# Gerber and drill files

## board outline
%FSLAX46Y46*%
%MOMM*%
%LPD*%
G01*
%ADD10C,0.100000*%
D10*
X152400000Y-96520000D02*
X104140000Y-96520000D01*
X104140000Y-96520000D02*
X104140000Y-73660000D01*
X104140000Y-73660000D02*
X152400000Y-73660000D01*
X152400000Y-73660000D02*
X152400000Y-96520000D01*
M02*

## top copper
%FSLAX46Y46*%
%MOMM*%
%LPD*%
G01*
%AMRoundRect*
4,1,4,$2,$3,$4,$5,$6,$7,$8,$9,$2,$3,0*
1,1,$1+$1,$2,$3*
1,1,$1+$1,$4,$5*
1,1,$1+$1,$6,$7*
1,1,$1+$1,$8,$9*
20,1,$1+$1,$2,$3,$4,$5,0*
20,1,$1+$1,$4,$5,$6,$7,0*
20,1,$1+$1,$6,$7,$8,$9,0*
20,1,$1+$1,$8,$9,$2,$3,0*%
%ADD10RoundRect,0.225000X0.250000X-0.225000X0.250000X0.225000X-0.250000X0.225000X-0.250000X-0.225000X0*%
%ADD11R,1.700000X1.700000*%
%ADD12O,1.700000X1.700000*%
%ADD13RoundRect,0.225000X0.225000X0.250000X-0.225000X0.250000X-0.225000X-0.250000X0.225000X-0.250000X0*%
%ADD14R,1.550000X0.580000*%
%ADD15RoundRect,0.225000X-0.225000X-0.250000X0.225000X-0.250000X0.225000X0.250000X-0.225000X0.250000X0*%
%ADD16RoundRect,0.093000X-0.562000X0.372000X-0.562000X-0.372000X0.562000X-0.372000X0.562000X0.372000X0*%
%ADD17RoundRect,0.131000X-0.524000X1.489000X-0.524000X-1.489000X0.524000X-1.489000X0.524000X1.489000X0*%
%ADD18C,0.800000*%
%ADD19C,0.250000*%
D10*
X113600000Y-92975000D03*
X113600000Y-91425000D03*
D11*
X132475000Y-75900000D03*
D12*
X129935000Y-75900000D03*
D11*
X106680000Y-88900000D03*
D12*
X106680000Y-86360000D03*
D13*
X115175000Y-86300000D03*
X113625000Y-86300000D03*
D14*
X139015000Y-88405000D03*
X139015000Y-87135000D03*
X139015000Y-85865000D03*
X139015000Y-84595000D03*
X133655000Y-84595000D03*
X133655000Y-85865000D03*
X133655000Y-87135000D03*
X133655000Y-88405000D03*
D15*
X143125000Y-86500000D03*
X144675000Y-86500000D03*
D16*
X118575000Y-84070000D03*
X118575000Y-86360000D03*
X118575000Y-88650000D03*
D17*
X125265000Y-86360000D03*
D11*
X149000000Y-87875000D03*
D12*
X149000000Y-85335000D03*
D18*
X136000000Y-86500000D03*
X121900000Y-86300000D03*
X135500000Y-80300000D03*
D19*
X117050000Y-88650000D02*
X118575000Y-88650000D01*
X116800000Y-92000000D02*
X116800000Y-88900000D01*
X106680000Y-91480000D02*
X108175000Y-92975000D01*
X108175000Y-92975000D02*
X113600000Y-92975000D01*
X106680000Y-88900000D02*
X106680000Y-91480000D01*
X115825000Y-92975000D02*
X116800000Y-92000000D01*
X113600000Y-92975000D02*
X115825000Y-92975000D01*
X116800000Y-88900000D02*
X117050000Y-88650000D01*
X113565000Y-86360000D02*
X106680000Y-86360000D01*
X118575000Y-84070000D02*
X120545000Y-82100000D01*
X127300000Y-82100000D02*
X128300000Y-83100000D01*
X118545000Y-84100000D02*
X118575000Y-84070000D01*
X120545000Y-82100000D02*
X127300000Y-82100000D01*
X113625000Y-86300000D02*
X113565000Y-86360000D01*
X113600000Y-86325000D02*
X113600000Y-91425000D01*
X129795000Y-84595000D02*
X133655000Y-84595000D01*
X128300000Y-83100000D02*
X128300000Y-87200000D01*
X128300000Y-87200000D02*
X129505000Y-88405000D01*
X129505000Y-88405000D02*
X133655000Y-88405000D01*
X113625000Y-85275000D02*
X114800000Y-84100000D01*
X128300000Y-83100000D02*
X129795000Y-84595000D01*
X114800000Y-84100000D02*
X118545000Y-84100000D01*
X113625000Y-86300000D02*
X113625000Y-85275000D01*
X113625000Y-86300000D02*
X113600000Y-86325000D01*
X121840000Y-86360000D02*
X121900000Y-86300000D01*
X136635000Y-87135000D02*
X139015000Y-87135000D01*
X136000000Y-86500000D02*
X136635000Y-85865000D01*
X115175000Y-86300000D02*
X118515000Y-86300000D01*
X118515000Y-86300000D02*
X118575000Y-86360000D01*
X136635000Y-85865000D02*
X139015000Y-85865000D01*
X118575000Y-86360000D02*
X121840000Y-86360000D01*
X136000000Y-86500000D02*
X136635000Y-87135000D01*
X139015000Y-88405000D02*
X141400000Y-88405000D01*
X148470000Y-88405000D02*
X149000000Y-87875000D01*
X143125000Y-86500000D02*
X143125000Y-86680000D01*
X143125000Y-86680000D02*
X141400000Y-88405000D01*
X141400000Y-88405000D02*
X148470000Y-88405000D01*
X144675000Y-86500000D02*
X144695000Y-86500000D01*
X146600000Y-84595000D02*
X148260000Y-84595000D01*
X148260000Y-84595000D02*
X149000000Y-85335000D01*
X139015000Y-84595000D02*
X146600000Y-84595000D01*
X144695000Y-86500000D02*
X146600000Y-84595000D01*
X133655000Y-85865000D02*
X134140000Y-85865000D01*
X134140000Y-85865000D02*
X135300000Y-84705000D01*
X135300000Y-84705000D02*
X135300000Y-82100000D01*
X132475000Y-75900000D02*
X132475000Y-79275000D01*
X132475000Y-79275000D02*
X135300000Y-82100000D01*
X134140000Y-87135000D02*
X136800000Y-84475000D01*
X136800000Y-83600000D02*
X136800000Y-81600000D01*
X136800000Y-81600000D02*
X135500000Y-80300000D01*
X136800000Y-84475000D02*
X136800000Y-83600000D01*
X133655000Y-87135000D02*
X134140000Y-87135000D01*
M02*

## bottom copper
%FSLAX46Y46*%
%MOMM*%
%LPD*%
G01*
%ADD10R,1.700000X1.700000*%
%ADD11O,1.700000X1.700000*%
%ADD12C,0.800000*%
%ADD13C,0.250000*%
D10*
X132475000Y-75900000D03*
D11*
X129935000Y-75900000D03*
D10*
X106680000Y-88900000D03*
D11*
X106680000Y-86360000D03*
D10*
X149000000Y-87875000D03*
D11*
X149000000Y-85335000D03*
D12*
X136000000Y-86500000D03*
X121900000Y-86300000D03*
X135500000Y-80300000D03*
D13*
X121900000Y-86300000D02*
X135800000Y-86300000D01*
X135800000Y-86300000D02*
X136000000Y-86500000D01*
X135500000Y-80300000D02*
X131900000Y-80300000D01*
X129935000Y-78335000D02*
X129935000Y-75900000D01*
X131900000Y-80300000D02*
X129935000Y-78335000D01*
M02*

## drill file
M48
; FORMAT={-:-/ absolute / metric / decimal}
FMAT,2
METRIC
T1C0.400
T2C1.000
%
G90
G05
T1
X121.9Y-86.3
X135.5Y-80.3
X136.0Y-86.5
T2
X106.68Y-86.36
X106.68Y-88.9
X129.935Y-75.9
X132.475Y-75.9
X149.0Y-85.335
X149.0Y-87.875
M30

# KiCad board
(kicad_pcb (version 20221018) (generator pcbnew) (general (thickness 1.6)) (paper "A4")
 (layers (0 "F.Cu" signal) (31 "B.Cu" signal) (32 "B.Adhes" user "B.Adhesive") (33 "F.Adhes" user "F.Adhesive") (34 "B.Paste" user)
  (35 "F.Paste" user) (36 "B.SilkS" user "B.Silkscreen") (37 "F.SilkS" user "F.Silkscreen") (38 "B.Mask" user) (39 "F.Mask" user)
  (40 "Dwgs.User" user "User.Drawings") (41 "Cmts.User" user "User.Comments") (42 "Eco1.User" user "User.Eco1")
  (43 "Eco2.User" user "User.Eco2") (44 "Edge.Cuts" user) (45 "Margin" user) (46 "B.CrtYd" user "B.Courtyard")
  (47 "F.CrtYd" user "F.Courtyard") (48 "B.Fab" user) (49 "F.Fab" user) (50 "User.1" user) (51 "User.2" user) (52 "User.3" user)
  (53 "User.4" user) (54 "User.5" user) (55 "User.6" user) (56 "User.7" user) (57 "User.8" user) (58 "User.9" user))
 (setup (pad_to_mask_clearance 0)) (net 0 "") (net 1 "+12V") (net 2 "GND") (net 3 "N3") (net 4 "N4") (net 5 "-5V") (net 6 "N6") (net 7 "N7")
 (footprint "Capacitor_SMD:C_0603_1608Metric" (layer "F.Cu") (at 113.6 92.2 90)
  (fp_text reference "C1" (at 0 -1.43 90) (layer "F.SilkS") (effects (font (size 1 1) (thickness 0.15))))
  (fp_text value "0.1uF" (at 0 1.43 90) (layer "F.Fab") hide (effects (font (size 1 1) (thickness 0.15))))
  (pad "1" smd roundrect (at -0.775 0 90) (size 0.9 0.95) (layers "F.Cu" "F.Paste" "F.Mask") (roundrect_rratio 0.25) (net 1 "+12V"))
  (pad "2" smd roundrect (at 0.775 0 90) (size 0.9 0.95) (layers "F.Cu" "F.Paste" "F.Mask") (roundrect_rratio 0.25) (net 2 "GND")))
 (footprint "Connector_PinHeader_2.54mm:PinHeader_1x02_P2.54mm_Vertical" (layer "F.Cu") (at 132.475 75.9 -90)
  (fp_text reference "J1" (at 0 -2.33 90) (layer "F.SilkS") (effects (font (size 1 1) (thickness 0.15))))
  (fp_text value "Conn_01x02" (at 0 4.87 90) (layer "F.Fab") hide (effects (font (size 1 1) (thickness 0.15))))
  (pad "1" thru_hole rect (at 0 0 270) (size 1.7 1.7) (drill 1) (layers "*.Cu" "*.Mask") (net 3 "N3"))
  (pad "2" thru_hole oval (at 0 2.54 270) (size 1.7 1.7) (drill 1) (layers "*.Cu" "*.Mask") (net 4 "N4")))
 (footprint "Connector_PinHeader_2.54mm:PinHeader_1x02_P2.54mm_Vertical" (layer "F.Cu") (at 106.68 88.9 180)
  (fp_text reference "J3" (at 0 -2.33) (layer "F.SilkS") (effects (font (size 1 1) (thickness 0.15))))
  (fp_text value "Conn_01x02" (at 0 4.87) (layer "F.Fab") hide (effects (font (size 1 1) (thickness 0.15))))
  (pad "1" thru_hole rect (at 0 0 180) (size 1.7 1.7) (drill 1) (layers "*.Cu" "*.Mask") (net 1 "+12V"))
  (pad "2" thru_hole oval (at 0 2.54 180) (size 1.7 1.7) (drill 1) (layers "*.Cu" "*.Mask") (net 2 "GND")))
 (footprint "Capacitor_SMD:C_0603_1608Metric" (layer "F.Cu") (at 114.4 86.3 180)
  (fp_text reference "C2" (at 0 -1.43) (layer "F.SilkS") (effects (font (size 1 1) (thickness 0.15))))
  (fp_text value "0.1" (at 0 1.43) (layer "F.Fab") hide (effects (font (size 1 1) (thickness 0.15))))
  (pad "1" smd roundrect (at -0.775 0 180) (size 0.9 0.95) (layers "F.Cu" "F.Paste" "F.Mask") (roundrect_rratio 0.25) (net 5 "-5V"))
  (pad "2" smd roundrect (at 0.775 0 180) (size 0.9 0.95) (layers "F.Cu" "F.Paste" "F.Mask") (roundrect_rratio 0.25) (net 2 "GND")))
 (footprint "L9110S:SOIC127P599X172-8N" (layer "F.Cu") (at 136.335 86.5 180)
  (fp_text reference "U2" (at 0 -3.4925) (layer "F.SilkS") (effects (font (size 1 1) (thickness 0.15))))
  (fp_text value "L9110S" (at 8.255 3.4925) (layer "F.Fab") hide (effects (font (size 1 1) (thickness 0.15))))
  (pad "1" smd rect (at -2.68 -1.905 180) (size 1.55 0.58) (layers "F.Cu" "F.Paste" "F.Mask") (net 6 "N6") (solder_mask_margin 0.102))
  (pad "2" smd rect (at -2.68 -0.635 180) (size 1.55 0.58) (layers "F.Cu" "F.Paste" "F.Mask") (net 5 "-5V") (solder_mask_margin 0.102))
  (pad "3" smd rect (at -2.68 0.635 180) (size 1.55 0.58) (layers "F.Cu" "F.Paste" "F.Mask") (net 5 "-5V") (solder_mask_margin 0.102))
  (pad "4" smd rect (at -2.68 1.905 180) (size 1.55 0.58) (layers "F.Cu" "F.Paste" "F.Mask") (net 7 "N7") (solder_mask_margin 0.102))
  (pad "5" smd rect (at 2.68 1.905 180) (size 1.55 0.58) (layers "F.Cu" "F.Paste" "F.Mask") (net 2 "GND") (solder_mask_margin 0.102))
  (pad "6" smd rect (at 2.68 0.635 180) (size 1.55 0.58) (layers "F.Cu" "F.Paste" "F.Mask") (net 3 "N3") (solder_mask_margin 0.102))
  (pad "7" smd rect (at 2.68 -0.635 180) (size 1.55 0.58) (layers "F.Cu" "F.Paste" "F.Mask") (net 4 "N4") (solder_mask_margin 0.102))
  (pad "8" smd rect (at 2.68 -1.905 180) (size 1.55 0.58) (layers "F.Cu" "F.Paste" "F.Mask") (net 2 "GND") (solder_mask_margin 0.102)))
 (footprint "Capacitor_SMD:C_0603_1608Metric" (layer "F.Cu") (at 143.9 86.5)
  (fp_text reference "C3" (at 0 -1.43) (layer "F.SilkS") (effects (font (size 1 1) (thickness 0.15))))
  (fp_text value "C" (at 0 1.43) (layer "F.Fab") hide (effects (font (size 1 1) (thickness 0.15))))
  (pad "1" smd roundrect (at -0.775 0) (size 0.9 0.95) (layers "F.Cu" "F.Paste" "F.Mask") (roundrect_rratio 0.25) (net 6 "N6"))
  (pad "2" smd roundrect (at 0.775 0) (size 0.9 0.95) (layers "F.Cu" "F.Paste" "F.Mask") (roundrect_rratio 0.25) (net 7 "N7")))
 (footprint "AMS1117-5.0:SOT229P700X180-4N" (layer "F.Cu") (at 121.92 86.36 -90)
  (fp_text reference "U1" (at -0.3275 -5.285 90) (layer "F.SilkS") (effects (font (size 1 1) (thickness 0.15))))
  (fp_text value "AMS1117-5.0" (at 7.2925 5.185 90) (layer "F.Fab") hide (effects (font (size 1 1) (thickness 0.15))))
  (pad "1" smd roundrect (at -2.29 3.345 270) (size 0.93 1.31) (layers "F.Cu" "F.Paste" "F.Mask") (roundrect_rratio 0.1) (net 2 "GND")
   (solder_mask_margin 0.102))
  (pad "2" smd roundrect (at 0 3.345 270) (size 0.93 1.31) (layers "F.Cu" "F.Paste" "F.Mask") (roundrect_rratio 0.1) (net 5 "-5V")
   (solder_mask_margin 0.102))
  (pad "3" smd roundrect (at 2.29 3.345 270) (size 0.93 1.31) (layers "F.Cu" "F.Paste" "F.Mask") (roundrect_rratio 0.1) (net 1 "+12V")
   (solder_mask_margin 0.102))
  (pad "4" smd roundrect (at 0 -3.345 270) (size 3.24 1.31) (layers "F.Cu" "F.Paste" "F.Mask") (roundrect_rratio 0.1)
   (solder_mask_margin 0.102)))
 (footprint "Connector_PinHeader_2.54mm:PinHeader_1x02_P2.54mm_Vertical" (layer "F.Cu") (at 149 87.875 180)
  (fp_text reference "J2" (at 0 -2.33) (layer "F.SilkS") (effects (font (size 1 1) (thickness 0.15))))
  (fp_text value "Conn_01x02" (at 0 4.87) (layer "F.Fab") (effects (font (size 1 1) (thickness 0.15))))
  (pad "1" thru_hole rect (at 0 0 180) (size 1.7 1.7) (drill 1) (layers "*.Cu" "*.Mask") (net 6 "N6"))
  (pad "2" thru_hole oval (at 0 2.54 180) (size 1.7 1.7) (drill 1) (layers "*.Cu" "*.Mask") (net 7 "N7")))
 (gr_line (start 152.4 96.52) (end 104.14 96.52) (stroke (width 0.1) (type default)) (layer "Edge.Cuts"))
 (gr_line (start 104.14 96.52) (end 104.14 73.66) (stroke (width 0.1) (type default)) (layer "Edge.Cuts"))
 (gr_line (start 104.14 73.66) (end 152.4 73.66) (stroke (width 0.1) (type default)) (layer "Edge.Cuts"))
 (gr_line (start 152.4 73.66) (end 152.4 96.52) (stroke (width 0.1) (type default)) (layer "Edge.Cuts"))
 (segment (start 117.05 88.65) (end 118.575 88.65) (width 0.25) (layer "F.Cu") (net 1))
 (segment (start 116.8 92) (end 116.8 88.9) (width 0.25) (layer "F.Cu") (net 1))
 (segment (start 106.68 91.48) (end 108.175 92.975) (width 0.25) (layer "F.Cu") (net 1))
 (segment (start 108.175 92.975) (end 113.6 92.975) (width 0.25) (layer "F.Cu") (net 1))
 (segment (start 106.68 88.9) (end 106.68 91.48) (width 0.25) (layer "F.Cu") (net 1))
 (segment (start 115.825 92.975) (end 116.8 92) (width 0.25) (layer "F.Cu") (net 1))
 (segment (start 113.6 92.975) (end 115.825 92.975) (width 0.25) (layer "F.Cu") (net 1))
 (segment (start 116.8 88.9) (end 117.05 88.65) (width 0.25) (layer "F.Cu") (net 1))
 (segment (start 113.565 86.36) (end 106.68 86.36) (width 0.25) (layer "F.Cu") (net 2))
 (segment (start 118.575 84.07) (end 120.545 82.1) (width 0.25) (layer "F.Cu") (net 2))
 (segment (start 127.3 82.1) (end 128.3 83.1) (width 0.25) (layer "F.Cu") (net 2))
 (segment (start 118.545 84.1) (end 118.575 84.07) (width 0.25) (layer "F.Cu") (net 2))
 (segment (start 120.545 82.1) (end 127.3 82.1) (width 0.25) (layer "F.Cu") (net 2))
 (segment (start 113.625 86.3) (end 113.565 86.36) (width 0.25) (layer "F.Cu") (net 2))
 (segment (start 113.6 86.325) (end 113.6 91.425) (width 0.25) (layer "F.Cu") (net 2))
 (segment (start 129.795 84.595) (end 133.655 84.595) (width 0.25) (layer "F.Cu") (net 2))
 (segment (start 128.3 83.1) (end 128.3 87.2) (width 0.25) (layer "F.Cu") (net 2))
 (segment (start 128.3 87.2) (end 129.505 88.405) (width 0.25) (layer "F.Cu") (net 2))
 (segment (start 129.505 88.405) (end 133.655 88.405) (width 0.25) (layer "F.Cu") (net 2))
 (segment (start 113.625 85.275) (end 114.8 84.1) (width 0.25) (layer "F.Cu") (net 2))
 (segment (start 128.3 83.1) (end 129.795 84.595) (width 0.25) (layer "F.Cu") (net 2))
 (segment (start 114.8 84.1) (end 118.545 84.1) (width 0.25) (layer "F.Cu") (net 2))
 (segment (start 113.625 86.3) (end 113.625 85.275) (width 0.25) (layer "F.Cu") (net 2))
 (segment (start 113.625 86.3) (end 113.6 86.325) (width 0.25) (layer "F.Cu") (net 2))
 (segment (start 121.84 86.36) (end 121.9 86.3) (width 0.25) (layer "F.Cu") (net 5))
 (segment (start 136.635 87.135) (end 139.015 87.135) (width 0.25) (layer "F.Cu") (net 5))
 (segment (start 136 86.5) (end 136.635 85.865) (width 0.25) (layer "F.Cu") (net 5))
 (segment (start 115.175 86.3) (end 118.515 86.3) (width 0.25) (layer "F.Cu") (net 5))
 (segment (start 118.515 86.3) (end 118.575 86.36) (width 0.25) (layer "F.Cu") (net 5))
 (segment (start 136.635 85.865) (end 139.015 85.865) (width 0.25) (layer "F.Cu") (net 5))
 (segment (start 118.575 86.36) (end 121.84 86.36) (width 0.25) (layer "F.Cu") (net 5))
 (segment (start 136 86.5) (end 136.635 87.135) (width 0.25) (layer "F.Cu") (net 5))
 (via (at 136 86.5) (size 0.8) (drill 0.4) (layers "F.Cu" "B.Cu") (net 5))
 (via (at 121.9 86.3) (size 0.8) (drill 0.4) (layers "F.Cu" "B.Cu") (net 5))
 (segment (start 121.9 86.3) (end 135.8 86.3) (width 0.25) (layer "B.Cu") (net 5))
 (segment (start 135.8 86.3) (end 136 86.5) (width 0.25) (layer "B.Cu") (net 5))
 (segment (start 139.015 88.405) (end 141.4 88.405) (width 0.25) (layer "F.Cu") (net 6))
 (segment (start 148.47 88.405) (end 149 87.875) (width 0.25) (layer "F.Cu") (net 6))
 (segment (start 143.125 86.5) (end 143.125 86.68) (width 0.25) (layer "F.Cu") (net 6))
 (segment (start 143.125 86.68) (end 141.4 88.405) (width 0.25) (layer "F.Cu") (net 6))
 (segment (start 141.4 88.405) (end 148.47 88.405) (width 0.25) (layer "F.Cu") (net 6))
 (segment (start 144.675 86.5) (end 144.695 86.5) (width 0.25) (layer "F.Cu") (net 7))
 (segment (start 146.6 84.595) (end 148.26 84.595) (width 0.25) (layer "F.Cu") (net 7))
 (segment (start 148.26 84.595) (end 149 85.335) (width 0.25) (layer "F.Cu") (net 7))
 (segment (start 139.015 84.595) (end 146.6 84.595) (width 0.25) (layer "F.Cu") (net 7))
 (segment (start 144.695 86.5) (end 146.6 84.595) (width 0.25) (layer "F.Cu") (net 7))
 (segment (start 133.655 85.865) (end 134.14 85.865) (width 0.25) (layer "F.Cu") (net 3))
 (segment (start 134.14 85.865) (end 135.3 84.705) (width 0.25) (layer "F.Cu") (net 3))
 (segment (start 135.3 84.705) (end 135.3 82.1) (width 0.25) (layer "F.Cu") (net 3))
 (segment (start 132.475 75.9) (end 132.475 79.275) (width 0.25) (layer "F.Cu") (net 3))
 (segment (start 132.475 79.275) (end 135.3 82.1) (width 0.25) (layer "F.Cu") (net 3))
 (segment (start 134.14 87.135) (end 136.8 84.475) (width 0.25) (layer "F.Cu") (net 4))
 (segment (start 136.8 83.6) (end 136.8 81.6) (width 0.25) (layer "F.Cu") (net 4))
 (segment (start 136.8 81.6) (end 135.5 80.3) (width 0.25) (layer "F.Cu") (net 4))
 (segment (start 136.8 84.475) (end 136.8 83.6) (width 0.25) (layer "F.Cu") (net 4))
 (segment (start 133.655 87.135) (end 134.14 87.135) (width 0.25) (layer "F.Cu") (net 4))
 (via (at 135.5 80.3) (size 0.8) (drill 0.4) (layers "F.Cu" "B.Cu") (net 4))
 (segment (start 135.5 80.3) (end 131.9 80.3) (width 0.25) (layer "B.Cu") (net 4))
 (segment (start 129.935 78.335) (end 129.935 75.9) (width 0.25) (layer "B.Cu") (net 4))
 (segment (start 131.9 80.3) (end 129.935 78.335) (width 0.25) (layer "B.Cu") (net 4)))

